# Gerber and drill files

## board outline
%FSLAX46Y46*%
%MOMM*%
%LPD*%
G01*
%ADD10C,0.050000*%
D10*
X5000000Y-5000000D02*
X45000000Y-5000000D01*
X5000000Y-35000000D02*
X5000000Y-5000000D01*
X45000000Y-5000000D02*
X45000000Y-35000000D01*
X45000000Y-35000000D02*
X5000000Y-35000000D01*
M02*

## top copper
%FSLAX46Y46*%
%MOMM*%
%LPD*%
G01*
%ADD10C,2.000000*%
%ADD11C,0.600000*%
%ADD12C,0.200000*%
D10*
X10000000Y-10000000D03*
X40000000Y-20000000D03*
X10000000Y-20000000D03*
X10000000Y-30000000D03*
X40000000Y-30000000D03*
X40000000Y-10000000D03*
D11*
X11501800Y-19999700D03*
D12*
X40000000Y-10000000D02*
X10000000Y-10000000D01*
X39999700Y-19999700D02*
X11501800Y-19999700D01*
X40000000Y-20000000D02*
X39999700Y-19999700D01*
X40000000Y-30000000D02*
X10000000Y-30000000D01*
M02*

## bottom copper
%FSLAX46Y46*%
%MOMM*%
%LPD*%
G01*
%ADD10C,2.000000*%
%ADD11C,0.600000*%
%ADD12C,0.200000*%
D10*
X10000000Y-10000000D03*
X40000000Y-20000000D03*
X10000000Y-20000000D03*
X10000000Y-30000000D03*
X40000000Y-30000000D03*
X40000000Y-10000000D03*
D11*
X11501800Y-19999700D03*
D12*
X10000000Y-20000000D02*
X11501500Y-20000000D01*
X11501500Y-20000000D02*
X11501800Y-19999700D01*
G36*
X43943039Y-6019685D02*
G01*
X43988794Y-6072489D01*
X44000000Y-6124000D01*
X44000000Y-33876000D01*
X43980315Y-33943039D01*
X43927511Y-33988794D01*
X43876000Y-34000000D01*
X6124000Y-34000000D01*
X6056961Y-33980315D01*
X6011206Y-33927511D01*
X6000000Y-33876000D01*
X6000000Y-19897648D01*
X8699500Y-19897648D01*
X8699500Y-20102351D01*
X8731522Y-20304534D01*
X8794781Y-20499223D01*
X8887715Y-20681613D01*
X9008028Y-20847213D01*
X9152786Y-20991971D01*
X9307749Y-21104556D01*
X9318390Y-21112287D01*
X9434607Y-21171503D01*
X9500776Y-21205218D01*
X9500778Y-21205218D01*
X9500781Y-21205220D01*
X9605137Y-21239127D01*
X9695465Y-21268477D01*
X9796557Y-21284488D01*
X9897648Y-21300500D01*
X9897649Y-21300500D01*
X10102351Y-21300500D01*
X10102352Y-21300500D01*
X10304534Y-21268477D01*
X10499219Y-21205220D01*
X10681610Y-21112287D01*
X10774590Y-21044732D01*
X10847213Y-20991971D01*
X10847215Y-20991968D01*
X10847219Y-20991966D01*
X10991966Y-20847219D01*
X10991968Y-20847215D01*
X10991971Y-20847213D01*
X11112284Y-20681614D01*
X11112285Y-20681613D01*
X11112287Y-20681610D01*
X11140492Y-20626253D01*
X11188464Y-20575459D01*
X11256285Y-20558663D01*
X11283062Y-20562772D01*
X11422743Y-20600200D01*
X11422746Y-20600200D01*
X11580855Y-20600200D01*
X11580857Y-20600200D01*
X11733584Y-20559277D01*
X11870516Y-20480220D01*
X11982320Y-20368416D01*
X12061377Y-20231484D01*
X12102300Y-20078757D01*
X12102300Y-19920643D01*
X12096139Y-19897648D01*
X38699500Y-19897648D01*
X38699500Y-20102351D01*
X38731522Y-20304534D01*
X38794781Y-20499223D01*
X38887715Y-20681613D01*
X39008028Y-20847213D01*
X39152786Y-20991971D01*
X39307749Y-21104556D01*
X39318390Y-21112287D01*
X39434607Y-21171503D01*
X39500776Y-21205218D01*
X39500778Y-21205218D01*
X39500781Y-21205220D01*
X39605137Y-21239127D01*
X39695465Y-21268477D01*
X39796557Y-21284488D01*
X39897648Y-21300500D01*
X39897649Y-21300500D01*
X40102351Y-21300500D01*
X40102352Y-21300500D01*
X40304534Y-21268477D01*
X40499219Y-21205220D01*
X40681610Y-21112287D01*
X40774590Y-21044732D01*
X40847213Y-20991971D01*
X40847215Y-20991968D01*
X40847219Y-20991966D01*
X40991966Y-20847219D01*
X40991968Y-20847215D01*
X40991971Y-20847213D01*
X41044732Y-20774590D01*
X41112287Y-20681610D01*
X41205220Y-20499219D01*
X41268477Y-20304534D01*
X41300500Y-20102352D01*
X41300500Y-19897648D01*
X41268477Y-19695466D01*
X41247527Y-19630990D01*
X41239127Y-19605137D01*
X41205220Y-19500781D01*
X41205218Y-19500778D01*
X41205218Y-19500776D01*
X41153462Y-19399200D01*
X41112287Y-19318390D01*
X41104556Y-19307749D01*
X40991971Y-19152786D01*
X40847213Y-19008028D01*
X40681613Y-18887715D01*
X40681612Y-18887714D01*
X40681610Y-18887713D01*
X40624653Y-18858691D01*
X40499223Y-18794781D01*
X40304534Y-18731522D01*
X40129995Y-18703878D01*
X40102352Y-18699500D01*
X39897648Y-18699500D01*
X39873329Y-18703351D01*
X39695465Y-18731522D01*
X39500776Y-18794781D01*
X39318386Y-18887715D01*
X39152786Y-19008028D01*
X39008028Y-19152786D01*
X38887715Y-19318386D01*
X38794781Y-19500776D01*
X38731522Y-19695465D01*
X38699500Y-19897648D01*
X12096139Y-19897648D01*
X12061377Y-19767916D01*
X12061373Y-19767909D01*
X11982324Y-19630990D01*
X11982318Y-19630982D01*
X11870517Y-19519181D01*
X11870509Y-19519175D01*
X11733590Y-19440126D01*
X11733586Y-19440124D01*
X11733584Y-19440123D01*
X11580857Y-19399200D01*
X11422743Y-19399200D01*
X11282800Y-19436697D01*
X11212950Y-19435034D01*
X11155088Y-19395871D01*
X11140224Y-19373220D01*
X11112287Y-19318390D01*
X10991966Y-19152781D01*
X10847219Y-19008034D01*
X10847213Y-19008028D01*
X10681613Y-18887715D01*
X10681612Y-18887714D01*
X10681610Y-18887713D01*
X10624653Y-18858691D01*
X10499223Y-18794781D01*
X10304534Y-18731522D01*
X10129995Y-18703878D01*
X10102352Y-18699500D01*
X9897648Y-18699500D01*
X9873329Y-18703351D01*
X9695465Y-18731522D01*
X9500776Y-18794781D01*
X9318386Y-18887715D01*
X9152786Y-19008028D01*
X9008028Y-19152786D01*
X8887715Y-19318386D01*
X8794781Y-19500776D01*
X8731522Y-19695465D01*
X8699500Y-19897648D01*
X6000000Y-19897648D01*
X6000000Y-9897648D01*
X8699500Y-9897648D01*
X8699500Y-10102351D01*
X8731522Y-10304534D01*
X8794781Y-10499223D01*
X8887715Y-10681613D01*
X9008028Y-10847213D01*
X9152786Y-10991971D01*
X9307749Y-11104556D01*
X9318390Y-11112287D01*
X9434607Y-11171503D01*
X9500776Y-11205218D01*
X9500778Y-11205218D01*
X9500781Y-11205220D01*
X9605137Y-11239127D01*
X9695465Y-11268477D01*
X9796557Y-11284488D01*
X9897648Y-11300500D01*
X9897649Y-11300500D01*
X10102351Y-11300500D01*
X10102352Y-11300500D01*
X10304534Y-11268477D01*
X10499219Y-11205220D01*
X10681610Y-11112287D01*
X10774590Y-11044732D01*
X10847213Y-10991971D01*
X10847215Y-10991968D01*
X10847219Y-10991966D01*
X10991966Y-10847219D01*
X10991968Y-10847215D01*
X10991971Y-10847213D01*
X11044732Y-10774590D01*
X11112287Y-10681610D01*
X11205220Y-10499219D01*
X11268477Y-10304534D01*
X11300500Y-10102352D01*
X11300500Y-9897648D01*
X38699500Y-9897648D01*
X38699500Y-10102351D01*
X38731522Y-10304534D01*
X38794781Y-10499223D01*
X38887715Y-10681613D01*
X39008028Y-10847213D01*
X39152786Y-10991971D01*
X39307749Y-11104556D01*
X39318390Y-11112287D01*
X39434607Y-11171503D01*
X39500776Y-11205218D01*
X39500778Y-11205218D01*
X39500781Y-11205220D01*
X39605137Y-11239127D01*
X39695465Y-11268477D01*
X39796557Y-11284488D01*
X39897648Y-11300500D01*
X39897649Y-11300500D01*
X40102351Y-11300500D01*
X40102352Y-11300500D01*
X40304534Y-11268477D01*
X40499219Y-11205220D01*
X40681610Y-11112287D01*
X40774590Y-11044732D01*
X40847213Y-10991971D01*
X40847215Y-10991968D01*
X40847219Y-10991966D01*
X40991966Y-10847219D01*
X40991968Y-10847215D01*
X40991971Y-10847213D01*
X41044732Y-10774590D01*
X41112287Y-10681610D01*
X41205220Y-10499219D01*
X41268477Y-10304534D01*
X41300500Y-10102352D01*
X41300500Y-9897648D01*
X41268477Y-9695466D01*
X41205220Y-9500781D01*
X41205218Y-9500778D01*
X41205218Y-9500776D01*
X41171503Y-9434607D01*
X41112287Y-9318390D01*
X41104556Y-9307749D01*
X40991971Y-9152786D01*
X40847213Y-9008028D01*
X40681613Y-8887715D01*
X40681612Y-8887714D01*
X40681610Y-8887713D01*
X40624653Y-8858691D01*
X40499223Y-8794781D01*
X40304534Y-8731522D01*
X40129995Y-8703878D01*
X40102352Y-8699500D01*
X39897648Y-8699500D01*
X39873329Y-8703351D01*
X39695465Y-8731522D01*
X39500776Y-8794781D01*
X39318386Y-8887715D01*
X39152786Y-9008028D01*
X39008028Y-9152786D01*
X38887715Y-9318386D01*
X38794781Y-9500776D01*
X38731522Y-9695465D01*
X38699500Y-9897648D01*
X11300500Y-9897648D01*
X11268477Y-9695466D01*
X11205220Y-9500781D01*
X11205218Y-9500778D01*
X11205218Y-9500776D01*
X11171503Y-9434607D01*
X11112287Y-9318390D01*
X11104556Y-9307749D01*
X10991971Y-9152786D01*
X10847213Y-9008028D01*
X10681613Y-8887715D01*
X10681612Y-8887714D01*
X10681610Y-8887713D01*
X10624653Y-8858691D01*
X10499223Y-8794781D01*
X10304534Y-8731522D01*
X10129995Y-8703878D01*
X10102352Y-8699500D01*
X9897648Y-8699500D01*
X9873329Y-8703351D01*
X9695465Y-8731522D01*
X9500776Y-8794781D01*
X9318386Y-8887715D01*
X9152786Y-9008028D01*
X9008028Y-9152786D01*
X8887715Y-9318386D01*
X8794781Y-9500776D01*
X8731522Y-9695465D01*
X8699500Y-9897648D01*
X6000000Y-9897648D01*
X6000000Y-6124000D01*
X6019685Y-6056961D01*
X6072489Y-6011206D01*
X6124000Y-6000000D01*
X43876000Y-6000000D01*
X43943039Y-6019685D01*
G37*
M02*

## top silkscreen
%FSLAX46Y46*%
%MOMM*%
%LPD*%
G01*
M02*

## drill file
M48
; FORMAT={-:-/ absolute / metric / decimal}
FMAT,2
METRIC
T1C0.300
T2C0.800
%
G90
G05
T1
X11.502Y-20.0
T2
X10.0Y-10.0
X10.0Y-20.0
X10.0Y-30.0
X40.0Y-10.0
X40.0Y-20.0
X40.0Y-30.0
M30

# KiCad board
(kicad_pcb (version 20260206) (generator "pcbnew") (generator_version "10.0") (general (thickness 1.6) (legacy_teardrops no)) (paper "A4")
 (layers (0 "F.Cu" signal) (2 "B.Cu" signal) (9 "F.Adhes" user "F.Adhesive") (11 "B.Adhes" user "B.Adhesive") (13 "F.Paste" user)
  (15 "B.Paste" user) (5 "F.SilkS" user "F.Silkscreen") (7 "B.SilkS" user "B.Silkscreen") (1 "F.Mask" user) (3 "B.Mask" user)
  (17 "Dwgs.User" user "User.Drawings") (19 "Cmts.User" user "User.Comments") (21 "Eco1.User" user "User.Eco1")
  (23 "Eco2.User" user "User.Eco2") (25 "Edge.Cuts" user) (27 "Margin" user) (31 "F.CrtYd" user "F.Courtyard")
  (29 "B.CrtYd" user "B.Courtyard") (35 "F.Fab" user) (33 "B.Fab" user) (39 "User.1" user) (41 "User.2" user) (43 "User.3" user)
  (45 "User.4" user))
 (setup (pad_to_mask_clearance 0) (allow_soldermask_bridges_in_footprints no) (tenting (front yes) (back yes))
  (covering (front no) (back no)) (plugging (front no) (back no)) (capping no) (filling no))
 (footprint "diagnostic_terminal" (layer "F.Cu") (at 10 10)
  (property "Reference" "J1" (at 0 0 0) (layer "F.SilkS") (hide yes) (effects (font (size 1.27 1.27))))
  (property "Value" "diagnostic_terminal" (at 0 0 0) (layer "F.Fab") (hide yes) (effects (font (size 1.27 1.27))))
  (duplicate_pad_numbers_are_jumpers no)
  (pad "1" thru_hole circle (at 0 0) (size 2 2) (drill 0.8) (layers "*.Cu") (remove_unused_layers no) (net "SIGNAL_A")))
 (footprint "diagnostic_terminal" (layer "F.Cu") (at 40 20)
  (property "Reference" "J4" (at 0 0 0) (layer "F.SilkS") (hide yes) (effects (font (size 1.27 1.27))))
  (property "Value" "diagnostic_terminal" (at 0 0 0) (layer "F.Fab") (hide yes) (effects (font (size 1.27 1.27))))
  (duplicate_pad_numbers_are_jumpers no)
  (pad "1" thru_hole circle (at 0 0) (size 2 2) (drill 0.8) (layers "*.Cu") (remove_unused_layers no) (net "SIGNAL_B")))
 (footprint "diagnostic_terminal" (layer "F.Cu") (at 10 20)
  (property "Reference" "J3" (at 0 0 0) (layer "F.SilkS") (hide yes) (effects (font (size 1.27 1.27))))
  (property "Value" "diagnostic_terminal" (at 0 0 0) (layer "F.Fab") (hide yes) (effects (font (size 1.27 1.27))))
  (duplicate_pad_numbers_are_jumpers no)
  (pad "1" thru_hole circle (at 0 0) (size 2 2) (drill 0.8) (layers "*.Cu") (remove_unused_layers no) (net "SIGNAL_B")))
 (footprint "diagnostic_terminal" (layer "F.Cu") (at 10 30)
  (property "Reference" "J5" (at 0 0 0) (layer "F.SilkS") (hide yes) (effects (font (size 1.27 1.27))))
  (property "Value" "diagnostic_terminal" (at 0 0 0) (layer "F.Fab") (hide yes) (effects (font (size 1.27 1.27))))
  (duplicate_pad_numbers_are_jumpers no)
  (pad "1" thru_hole circle (at 0 0) (size 2 2) (drill 0.8) (layers "*.Cu") (remove_unused_layers no) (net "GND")))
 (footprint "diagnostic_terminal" (layer "F.Cu") (at 40 30)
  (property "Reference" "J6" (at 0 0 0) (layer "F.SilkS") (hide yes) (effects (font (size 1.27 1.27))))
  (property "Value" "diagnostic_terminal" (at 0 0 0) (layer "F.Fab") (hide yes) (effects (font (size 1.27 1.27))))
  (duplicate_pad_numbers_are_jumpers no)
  (pad "1" thru_hole circle (at 0 0) (size 2 2) (drill 0.8) (layers "*.Cu") (remove_unused_layers no) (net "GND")))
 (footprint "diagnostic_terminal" (layer "F.Cu") (at 40 10)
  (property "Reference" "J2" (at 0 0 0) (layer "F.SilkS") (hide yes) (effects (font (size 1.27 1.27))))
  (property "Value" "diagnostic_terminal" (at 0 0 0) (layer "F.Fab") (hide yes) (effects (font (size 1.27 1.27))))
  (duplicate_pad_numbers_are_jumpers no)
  (pad "1" thru_hole circle (at 0 0) (size 2 2) (drill 0.8) (layers "*.Cu") (remove_unused_layers no) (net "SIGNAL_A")))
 (gr_line (start 5 5) (end 45 5) (stroke (width 0.05) (type default)) (layer "Edge.Cuts"))
 (gr_line (start 5 35) (end 5 5) (stroke (width 0.05) (type default)) (layer "Edge.Cuts"))
 (gr_line (start 45 5) (end 45 35) (stroke (width 0.05) (type default)) (layer "Edge.Cuts"))
 (gr_line (start 45 35) (end 5 35) (stroke (width 0.05) (type default)) (layer "Edge.Cuts"))
 (segment (start 40 10) (end 10 10) (width 0.2) (layer "F.Cu") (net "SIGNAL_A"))
 (segment (start 39.9997 19.9997) (end 11.5018 19.9997) (width 0.2) (layer "F.Cu") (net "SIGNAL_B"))
 (segment (start 40 20) (end 39.9997 19.9997) (width 0.2) (layer "F.Cu") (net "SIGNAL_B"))
 (via (at 11.5018 19.9997) (size 0.6) (drill 0.3) (layers "F.Cu" "B.Cu") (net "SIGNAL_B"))
 (segment (start 10 20) (end 11.5015 20) (width 0.2) (layer "B.Cu") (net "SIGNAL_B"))
 (segment (start 11.5015 20) (end 11.5018 19.9997) (width 0.2) (layer "B.Cu") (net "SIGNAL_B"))
 (segment (start 40 30) (end 10 30) (width 0.2) (layer "F.Cu") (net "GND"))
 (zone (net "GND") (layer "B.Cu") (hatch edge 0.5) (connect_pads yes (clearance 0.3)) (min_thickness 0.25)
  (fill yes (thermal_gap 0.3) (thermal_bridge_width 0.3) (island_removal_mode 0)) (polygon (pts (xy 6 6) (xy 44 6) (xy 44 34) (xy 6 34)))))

